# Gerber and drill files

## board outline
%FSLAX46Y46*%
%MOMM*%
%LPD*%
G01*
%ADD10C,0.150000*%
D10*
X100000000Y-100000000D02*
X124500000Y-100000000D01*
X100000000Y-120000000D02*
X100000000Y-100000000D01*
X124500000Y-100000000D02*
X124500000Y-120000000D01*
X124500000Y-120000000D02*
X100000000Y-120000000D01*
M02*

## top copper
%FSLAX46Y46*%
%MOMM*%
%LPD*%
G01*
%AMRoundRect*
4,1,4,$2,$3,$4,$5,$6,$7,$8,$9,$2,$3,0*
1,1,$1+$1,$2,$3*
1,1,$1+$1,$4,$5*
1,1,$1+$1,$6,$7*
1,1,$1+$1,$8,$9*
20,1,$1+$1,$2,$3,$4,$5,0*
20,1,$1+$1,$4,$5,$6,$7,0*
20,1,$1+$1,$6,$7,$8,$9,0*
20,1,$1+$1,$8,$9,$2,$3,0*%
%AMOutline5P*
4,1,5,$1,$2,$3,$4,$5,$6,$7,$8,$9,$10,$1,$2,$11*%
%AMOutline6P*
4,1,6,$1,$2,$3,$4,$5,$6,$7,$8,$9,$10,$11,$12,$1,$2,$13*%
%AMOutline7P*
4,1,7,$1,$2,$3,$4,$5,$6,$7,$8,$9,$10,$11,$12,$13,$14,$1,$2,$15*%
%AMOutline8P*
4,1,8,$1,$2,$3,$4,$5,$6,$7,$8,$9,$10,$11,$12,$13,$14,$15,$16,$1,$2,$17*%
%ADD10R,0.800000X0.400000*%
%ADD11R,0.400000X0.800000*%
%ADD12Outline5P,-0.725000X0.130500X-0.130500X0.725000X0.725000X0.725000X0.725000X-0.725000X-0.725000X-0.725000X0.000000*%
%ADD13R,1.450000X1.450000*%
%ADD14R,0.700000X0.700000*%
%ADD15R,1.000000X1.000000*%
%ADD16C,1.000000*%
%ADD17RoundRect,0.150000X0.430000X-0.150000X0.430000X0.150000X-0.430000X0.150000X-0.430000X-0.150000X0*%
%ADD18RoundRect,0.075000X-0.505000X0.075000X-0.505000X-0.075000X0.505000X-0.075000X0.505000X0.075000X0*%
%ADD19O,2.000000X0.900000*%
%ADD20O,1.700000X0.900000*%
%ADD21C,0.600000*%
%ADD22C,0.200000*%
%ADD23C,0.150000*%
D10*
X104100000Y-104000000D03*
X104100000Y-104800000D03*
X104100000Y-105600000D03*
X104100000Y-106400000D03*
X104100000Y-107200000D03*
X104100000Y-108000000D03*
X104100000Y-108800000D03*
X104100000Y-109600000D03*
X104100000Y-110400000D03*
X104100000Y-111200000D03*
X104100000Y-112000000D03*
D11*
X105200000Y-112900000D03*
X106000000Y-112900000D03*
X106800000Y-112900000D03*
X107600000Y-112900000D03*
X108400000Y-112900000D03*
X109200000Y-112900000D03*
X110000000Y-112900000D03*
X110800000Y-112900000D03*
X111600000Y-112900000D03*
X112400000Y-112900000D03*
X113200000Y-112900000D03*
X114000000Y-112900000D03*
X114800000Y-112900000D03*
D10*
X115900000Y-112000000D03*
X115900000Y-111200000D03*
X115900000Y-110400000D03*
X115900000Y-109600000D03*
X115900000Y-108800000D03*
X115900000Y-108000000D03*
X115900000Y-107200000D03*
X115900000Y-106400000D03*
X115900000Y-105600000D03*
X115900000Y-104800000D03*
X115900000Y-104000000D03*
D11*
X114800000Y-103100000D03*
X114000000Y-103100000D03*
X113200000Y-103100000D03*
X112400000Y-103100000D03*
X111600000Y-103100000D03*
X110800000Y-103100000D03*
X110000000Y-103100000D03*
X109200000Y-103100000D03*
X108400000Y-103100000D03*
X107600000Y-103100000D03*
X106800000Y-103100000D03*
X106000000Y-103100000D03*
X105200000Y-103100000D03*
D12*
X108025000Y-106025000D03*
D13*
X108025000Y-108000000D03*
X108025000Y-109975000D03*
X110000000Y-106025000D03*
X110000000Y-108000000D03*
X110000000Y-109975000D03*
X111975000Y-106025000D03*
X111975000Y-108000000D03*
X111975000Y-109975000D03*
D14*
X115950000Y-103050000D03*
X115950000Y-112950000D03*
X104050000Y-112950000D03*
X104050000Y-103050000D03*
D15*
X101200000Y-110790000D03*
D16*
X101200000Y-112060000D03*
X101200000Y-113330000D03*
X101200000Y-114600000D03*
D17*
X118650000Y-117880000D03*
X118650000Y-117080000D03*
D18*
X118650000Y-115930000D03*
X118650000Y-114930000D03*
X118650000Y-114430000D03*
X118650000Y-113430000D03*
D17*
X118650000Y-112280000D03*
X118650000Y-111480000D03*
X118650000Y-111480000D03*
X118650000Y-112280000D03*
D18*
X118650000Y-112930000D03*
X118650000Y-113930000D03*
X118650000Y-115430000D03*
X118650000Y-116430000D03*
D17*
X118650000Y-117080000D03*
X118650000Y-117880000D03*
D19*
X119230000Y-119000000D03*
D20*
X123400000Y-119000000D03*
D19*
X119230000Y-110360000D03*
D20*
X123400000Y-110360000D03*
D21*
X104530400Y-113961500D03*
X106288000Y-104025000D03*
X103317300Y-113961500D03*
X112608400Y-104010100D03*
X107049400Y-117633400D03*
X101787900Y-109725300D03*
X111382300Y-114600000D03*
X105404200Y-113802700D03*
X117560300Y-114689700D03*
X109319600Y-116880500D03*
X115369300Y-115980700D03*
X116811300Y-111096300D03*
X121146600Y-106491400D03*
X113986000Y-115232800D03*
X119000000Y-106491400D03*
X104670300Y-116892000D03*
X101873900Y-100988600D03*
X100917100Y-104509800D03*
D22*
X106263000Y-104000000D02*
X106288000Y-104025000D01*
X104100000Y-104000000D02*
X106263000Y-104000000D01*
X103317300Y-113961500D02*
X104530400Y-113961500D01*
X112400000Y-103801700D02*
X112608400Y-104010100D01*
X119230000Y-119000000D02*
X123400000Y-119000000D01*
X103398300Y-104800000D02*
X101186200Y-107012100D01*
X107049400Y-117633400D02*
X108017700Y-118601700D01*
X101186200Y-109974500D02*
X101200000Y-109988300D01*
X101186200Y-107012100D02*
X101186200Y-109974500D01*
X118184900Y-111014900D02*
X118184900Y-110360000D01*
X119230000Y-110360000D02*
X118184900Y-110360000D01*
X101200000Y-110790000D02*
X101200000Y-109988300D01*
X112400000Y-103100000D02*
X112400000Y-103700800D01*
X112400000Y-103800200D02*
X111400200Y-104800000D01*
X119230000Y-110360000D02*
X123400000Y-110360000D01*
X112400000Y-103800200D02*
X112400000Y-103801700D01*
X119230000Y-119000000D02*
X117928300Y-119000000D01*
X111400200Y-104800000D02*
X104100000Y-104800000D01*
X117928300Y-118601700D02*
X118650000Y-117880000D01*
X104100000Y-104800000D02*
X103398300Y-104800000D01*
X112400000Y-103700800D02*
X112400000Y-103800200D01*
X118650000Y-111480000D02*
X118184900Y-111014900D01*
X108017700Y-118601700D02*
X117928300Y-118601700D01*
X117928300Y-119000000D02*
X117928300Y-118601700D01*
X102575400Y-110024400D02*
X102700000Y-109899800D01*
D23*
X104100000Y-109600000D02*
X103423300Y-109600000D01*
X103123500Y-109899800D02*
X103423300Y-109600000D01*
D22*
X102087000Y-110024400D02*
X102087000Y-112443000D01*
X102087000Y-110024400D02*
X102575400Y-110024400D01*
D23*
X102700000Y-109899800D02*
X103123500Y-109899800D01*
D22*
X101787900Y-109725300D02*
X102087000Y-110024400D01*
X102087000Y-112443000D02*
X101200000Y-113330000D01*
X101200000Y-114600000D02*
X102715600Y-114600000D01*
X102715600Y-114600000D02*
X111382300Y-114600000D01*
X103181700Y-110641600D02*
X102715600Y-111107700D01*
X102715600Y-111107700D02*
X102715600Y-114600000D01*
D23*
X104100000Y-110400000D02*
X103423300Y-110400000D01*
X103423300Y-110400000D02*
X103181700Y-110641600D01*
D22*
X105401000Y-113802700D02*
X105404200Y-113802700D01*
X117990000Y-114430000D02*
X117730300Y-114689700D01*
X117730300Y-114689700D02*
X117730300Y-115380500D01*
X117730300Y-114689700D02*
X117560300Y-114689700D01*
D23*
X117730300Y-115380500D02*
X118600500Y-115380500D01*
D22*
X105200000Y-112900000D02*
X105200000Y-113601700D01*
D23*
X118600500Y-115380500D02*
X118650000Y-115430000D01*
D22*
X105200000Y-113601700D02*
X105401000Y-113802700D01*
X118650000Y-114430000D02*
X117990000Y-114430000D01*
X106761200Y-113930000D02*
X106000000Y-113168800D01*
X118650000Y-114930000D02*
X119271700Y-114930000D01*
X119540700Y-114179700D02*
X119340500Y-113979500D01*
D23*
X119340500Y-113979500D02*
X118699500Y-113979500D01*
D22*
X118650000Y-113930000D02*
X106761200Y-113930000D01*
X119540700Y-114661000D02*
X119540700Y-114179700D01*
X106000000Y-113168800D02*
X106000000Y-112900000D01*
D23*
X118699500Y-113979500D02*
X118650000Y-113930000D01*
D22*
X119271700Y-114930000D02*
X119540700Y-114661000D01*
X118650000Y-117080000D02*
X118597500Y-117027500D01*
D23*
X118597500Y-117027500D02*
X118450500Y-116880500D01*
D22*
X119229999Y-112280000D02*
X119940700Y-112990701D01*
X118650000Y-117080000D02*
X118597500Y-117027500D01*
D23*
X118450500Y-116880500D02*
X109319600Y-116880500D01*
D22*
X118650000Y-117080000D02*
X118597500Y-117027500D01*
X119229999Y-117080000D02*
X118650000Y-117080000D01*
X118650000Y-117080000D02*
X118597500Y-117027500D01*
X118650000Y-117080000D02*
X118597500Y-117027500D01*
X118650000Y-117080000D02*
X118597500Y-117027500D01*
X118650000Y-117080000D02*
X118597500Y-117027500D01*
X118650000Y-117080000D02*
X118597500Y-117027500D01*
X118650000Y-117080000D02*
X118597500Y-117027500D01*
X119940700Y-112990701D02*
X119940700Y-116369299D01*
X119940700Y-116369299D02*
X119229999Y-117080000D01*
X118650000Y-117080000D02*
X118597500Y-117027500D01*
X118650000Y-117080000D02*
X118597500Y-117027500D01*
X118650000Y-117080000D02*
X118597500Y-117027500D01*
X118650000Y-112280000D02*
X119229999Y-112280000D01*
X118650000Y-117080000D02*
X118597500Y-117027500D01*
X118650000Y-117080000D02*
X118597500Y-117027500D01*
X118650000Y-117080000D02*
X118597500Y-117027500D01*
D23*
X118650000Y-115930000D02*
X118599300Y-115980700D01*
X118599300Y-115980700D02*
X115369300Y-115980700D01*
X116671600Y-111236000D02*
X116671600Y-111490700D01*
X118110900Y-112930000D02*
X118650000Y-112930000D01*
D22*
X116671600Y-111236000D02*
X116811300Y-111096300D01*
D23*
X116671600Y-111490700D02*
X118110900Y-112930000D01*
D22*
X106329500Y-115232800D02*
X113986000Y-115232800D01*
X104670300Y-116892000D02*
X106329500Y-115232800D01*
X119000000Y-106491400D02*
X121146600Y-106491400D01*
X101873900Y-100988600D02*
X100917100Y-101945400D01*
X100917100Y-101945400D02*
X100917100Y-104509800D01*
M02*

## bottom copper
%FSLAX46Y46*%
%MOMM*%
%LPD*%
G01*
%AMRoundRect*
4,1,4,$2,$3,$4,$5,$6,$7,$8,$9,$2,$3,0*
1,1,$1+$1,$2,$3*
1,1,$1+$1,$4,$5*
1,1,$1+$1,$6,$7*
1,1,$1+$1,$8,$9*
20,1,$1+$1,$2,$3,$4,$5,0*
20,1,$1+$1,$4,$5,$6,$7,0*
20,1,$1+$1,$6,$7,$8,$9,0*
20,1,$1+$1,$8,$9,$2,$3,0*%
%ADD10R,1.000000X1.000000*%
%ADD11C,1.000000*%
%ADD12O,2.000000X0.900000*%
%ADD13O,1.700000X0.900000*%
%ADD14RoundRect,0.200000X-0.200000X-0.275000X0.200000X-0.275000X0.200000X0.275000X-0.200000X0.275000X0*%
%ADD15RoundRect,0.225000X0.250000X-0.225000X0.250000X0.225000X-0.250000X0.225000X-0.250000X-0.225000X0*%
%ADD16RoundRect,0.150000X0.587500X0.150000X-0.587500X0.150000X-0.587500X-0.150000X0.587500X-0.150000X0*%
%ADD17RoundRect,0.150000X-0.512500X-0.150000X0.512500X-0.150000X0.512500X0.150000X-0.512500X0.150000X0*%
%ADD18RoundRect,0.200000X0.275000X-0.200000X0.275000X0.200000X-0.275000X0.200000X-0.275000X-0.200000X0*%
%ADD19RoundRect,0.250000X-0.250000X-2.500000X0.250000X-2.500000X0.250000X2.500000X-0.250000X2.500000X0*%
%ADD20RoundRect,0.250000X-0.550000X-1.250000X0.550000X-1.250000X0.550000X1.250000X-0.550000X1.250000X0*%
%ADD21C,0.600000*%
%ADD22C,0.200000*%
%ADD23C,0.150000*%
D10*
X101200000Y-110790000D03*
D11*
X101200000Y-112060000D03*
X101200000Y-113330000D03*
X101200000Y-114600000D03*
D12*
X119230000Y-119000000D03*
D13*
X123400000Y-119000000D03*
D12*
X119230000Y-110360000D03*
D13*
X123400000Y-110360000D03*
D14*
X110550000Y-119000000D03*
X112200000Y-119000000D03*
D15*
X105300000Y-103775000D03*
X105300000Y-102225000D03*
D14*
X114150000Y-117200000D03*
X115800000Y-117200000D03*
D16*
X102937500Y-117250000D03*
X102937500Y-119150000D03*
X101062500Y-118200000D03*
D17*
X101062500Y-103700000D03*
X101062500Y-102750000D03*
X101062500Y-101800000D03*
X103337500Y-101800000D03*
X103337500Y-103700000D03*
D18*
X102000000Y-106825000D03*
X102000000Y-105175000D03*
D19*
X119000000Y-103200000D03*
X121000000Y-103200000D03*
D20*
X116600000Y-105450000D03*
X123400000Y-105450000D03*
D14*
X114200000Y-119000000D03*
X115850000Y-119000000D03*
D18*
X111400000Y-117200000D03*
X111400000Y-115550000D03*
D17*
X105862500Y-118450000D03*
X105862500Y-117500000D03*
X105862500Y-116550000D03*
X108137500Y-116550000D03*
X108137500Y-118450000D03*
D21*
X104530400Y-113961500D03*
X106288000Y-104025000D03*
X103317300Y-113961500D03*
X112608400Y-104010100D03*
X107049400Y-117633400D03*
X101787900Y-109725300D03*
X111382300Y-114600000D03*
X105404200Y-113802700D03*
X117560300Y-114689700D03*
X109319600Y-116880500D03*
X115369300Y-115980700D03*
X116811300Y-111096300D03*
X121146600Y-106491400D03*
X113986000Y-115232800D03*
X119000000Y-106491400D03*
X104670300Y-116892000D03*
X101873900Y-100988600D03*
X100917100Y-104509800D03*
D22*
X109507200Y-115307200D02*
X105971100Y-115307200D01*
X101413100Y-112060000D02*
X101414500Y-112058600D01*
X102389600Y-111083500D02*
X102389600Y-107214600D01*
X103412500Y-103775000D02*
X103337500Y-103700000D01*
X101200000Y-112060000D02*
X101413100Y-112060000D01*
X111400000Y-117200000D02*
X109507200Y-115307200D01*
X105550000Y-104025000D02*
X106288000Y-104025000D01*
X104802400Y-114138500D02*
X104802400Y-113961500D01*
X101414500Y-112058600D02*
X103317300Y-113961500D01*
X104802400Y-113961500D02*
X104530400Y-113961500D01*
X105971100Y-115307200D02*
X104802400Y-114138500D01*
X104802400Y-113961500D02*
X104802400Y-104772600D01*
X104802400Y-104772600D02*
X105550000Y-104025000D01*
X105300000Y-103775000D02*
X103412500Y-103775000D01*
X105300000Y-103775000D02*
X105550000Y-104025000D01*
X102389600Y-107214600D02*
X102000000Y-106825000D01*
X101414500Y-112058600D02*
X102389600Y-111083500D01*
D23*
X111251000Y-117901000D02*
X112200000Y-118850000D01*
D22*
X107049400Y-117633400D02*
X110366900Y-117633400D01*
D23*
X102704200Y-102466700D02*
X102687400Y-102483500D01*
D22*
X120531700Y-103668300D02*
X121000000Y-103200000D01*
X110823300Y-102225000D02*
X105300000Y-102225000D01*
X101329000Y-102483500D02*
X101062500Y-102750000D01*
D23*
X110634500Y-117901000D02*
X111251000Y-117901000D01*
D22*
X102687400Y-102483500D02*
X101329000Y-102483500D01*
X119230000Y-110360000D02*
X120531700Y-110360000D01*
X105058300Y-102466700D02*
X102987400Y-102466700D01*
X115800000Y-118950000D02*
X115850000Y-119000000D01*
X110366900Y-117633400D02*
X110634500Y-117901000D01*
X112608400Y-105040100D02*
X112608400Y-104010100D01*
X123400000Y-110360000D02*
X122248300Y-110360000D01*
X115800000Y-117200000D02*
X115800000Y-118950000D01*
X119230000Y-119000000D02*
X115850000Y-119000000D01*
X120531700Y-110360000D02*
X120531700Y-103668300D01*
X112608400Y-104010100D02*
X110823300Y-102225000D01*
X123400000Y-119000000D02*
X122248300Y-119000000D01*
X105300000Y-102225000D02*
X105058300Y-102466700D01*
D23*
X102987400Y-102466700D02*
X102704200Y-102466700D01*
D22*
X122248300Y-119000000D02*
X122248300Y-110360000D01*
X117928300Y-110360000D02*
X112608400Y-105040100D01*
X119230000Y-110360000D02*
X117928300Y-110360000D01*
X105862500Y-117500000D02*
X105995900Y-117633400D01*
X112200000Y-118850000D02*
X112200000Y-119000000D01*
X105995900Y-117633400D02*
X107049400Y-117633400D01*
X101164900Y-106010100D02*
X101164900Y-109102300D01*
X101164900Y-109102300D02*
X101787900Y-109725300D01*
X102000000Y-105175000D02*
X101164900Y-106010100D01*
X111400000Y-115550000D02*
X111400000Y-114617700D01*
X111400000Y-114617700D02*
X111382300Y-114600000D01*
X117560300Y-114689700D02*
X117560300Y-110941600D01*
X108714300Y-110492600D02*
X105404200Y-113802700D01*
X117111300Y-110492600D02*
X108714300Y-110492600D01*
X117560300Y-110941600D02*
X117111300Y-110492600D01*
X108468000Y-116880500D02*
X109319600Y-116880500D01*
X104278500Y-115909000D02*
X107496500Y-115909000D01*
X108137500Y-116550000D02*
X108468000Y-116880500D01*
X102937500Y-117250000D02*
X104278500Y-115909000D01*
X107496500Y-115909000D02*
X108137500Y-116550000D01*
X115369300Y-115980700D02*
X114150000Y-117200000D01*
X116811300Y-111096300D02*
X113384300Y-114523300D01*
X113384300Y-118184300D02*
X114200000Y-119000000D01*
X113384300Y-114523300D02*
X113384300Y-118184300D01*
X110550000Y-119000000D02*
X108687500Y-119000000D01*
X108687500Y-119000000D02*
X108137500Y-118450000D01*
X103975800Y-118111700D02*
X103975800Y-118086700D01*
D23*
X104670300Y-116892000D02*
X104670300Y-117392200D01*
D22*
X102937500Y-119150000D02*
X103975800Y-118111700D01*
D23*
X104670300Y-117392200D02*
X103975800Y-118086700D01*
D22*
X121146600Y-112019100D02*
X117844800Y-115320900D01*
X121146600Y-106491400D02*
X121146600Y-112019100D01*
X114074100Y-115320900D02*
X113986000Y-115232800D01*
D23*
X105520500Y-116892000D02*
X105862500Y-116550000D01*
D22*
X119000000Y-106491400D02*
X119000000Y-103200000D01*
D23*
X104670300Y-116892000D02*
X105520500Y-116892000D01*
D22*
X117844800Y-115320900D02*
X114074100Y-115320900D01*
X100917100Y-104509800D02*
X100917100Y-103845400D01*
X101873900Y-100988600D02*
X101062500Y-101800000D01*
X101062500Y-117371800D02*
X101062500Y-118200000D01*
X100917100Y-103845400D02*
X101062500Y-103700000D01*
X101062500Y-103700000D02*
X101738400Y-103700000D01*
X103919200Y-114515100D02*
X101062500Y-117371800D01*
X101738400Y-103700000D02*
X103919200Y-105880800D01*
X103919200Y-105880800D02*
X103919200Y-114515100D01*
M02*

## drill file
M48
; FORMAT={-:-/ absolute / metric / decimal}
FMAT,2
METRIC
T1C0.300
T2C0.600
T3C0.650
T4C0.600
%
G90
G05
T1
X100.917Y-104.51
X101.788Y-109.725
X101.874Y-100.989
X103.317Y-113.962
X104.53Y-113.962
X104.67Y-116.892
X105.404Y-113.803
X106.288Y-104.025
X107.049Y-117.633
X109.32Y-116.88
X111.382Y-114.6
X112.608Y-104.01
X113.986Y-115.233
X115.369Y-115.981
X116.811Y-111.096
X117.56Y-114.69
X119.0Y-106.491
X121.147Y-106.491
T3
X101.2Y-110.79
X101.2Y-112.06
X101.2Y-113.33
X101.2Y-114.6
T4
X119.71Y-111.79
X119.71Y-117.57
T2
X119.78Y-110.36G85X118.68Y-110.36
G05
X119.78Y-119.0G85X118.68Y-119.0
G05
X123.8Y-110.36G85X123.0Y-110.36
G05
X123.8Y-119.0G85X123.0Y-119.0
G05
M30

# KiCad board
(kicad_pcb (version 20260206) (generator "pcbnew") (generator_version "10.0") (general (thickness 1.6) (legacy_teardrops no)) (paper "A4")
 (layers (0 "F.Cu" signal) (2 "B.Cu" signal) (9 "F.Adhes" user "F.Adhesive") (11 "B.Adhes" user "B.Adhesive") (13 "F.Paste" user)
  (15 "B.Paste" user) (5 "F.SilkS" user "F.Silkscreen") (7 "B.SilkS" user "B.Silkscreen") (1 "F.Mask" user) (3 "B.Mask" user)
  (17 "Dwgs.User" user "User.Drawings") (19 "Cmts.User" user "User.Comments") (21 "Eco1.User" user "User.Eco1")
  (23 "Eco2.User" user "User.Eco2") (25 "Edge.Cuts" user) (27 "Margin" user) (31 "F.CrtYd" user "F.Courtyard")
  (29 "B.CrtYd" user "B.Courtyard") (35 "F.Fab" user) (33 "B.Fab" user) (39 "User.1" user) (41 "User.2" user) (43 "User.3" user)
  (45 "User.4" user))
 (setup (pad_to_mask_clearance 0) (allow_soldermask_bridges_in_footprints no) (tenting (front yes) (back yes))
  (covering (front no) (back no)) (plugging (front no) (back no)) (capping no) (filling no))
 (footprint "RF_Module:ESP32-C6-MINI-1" (layer "F.Cu") (at 110 108)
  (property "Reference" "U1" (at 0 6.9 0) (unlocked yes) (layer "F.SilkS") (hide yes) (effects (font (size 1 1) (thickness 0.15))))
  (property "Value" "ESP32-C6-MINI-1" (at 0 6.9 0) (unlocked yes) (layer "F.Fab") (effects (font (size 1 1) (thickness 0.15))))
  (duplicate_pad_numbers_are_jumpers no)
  (pad "1" smd rect (at -5.9 -4) (size 0.8 0.4) (layers "F.Cu" "F.Mask" "F.Paste") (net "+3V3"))
  (pad "2" smd rect (at -5.9 -3.2) (size 0.8 0.4) (layers "F.Cu" "F.Mask" "F.Paste") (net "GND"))
  (pad "3" smd rect (at -5.9 -2.4) (size 0.8 0.4) (layers "F.Cu" "F.Mask" "F.Paste"))
  (pad "4" smd rect (at -5.9 -1.6) (size 0.8 0.4) (layers "F.Cu" "F.Mask" "F.Paste"))
  (pad "5" smd rect (at -5.9 -0.8) (size 0.8 0.4) (layers "F.Cu" "F.Mask" "F.Paste"))
  (pad "6" smd rect (at -5.9 0) (size 0.8 0.4) (layers "F.Cu" "F.Mask" "F.Paste"))
  (pad "7" smd rect (at -5.9 0.8) (size 0.8 0.4) (layers "F.Cu" "F.Mask" "F.Paste"))
  (pad "8" smd rect (at -5.9 1.6) (size 0.8 0.4) (layers "F.Cu" "F.Mask" "F.Paste") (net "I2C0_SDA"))
  (pad "9" smd rect (at -5.9 2.4) (size 0.8 0.4) (layers "F.Cu" "F.Mask" "F.Paste") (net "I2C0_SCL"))
  (pad "10" smd rect (at -5.9 3.2) (size 0.8 0.4) (layers "F.Cu" "F.Mask" "F.Paste"))
  (pad "11" smd rect (at -5.9 4) (size 0.8 0.4) (layers "F.Cu" "F.Mask" "F.Paste"))
  (pad "12" smd rect (at -4.8 4.9 90) (size 0.8 0.4) (layers "F.Cu" "F.Mask" "F.Paste") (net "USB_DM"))
  (pad "13" smd rect (at -4 4.9 90) (size 0.8 0.4) (layers "F.Cu" "F.Mask" "F.Paste") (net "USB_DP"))
  (pad "14" smd rect (at -3.2 4.9 90) (size 0.8 0.4) (layers "F.Cu" "F.Mask" "F.Paste"))
  (pad "15" smd rect (at -2.4 4.9 90) (size 0.8 0.4) (layers "F.Cu" "F.Mask" "F.Paste"))
  (pad "16" smd rect (at -1.6 4.9 90) (size 0.8 0.4) (layers "F.Cu" "F.Mask" "F.Paste"))
  (pad "17" smd rect (at -0.8 4.9 90) (size 0.8 0.4) (layers "F.Cu" "F.Mask" "F.Paste"))
  (pad "18" smd rect (at 0 4.9 90) (size 0.8 0.4) (layers "F.Cu" "F.Mask" "F.Paste"))
  (pad "19" smd rect (at 0.8 4.9 90) (size 0.8 0.4) (layers "F.Cu" "F.Mask" "F.Paste"))
  (pad "20" smd rect (at 1.6 4.9 90) (size 0.8 0.4) (layers "F.Cu" "F.Mask" "F.Paste"))
  (pad "21" smd rect (at 2.4 4.9 90) (size 0.8 0.4) (layers "F.Cu" "F.Mask" "F.Paste"))
  (pad "22" smd rect (at 3.2 4.9 90) (size 0.8 0.4) (layers "F.Cu" "F.Mask" "F.Paste"))
  (pad "23" smd rect (at 4 4.9 90) (size 0.8 0.4) (layers "F.Cu" "F.Mask" "F.Paste"))
  (pad "24" smd rect (at 4.8 4.9 90) (size 0.8 0.4) (layers "F.Cu" "F.Mask" "F.Paste"))
  (pad "25" smd rect (at 5.9 4) (size 0.8 0.4) (layers "F.Cu" "F.Mask" "F.Paste"))
  (pad "26" smd rect (at 5.9 3.2) (size 0.8 0.4) (layers "F.Cu" "F.Mask" "F.Paste"))
  (pad "27" smd rect (at 5.9 2.4) (size 0.8 0.4) (layers "F.Cu" "F.Mask" "F.Paste"))
  (pad "28" smd rect (at 5.9 1.6) (size 0.8 0.4) (layers "F.Cu" "F.Mask" "F.Paste"))
  (pad "29" smd rect (at 5.9 0.8) (size 0.8 0.4) (layers "F.Cu" "F.Mask" "F.Paste"))
  (pad "30" smd rect (at 5.9 0) (size 0.8 0.4) (layers "F.Cu" "F.Mask" "F.Paste"))
  (pad "31" smd rect (at 5.9 -0.8) (size 0.8 0.4) (layers "F.Cu" "F.Mask" "F.Paste"))
  (pad "32" smd rect (at 5.9 -1.6) (size 0.8 0.4) (layers "F.Cu" "F.Mask" "F.Paste"))
  (pad "33" smd rect (at 5.9 -2.4) (size 0.8 0.4) (layers "F.Cu" "F.Mask" "F.Paste"))
  (pad "34" smd rect (at 5.9 -3.2) (size 0.8 0.4) (layers "F.Cu" "F.Mask" "F.Paste"))
  (pad "35" smd rect (at 5.9 -4) (size 0.8 0.4) (layers "F.Cu" "F.Mask" "F.Paste"))
  (pad "36" smd rect (at 4.8 -4.9 90) (size 0.8 0.4) (layers "F.Cu" "F.Mask" "F.Paste"))
  (pad "37" smd rect (at 4 -4.9 90) (size 0.8 0.4) (layers "F.Cu" "F.Mask" "F.Paste"))
  (pad "38" smd rect (at 3.2 -4.9 90) (size 0.8 0.4) (layers "F.Cu" "F.Mask" "F.Paste"))
  (pad "39" smd rect (at 2.4 -4.9 90) (size 0.8 0.4) (layers "F.Cu" "F.Mask" "F.Paste") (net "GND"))
  (pad "40" smd rect (at 1.6 -4.9 90) (size 0.8 0.4) (layers "F.Cu" "F.Mask" "F.Paste"))
  (pad "41" smd rect (at 0.8 -4.9 90) (size 0.8 0.4) (layers "F.Cu" "F.Mask" "F.Paste"))
  (pad "42" smd rect (at 0 -4.9 90) (size 0.8 0.4) (layers "F.Cu" "F.Mask" "F.Paste"))
  (pad "43" smd rect (at -0.8 -4.9 90) (size 0.8 0.4) (layers "F.Cu" "F.Mask" "F.Paste"))
  (pad "44" smd rect (at -1.6 -4.9 90) (size 0.8 0.4) (layers "F.Cu" "F.Mask" "F.Paste"))
  (pad "45" smd rect (at -2.4 -4.9 90) (size 0.8 0.4) (layers "F.Cu" "F.Mask" "F.Paste"))
  (pad "46" smd rect (at -3.2 -4.9 90) (size 0.8 0.4) (layers "F.Cu" "F.Mask" "F.Paste"))
  (pad "47" smd rect (at -4 -4.9 90) (size 0.8 0.4) (layers "F.Cu" "F.Mask" "F.Paste"))
  (pad "48" smd rect (at -4.8 -4.9 90) (size 0.8 0.4) (layers "F.Cu" "F.Mask" "F.Paste"))
  (pad "49" smd roundrect (at -1.975 -1.975) (size 1.45 1.45) (layers "F.Cu" "F.Mask" "F.Paste") (roundrect_rratio 0) (chamfer_ratio 0.41)
   (chamfer top_left) (zone_connect 2))
  (pad "49" smd rect (at -1.975 0) (size 1.45 1.45) (layers "F.Cu" "F.Mask" "F.Paste") (zone_connect 2))
  (pad "49" smd rect (at -1.975 1.975) (size 1.45 1.45) (layers "F.Cu" "F.Mask" "F.Paste") (zone_connect 2))
  (pad "49" smd rect (at 0 -1.975) (size 1.45 1.45) (layers "F.Cu" "F.Mask" "F.Paste") (zone_connect 2))
  (pad "49" smd rect (at 0 0) (size 1.45 1.45) (layers "F.Cu" "F.Mask" "F.Paste") (zone_connect 2))
  (pad "49" smd rect (at 0 1.975) (size 1.45 1.45) (layers "F.Cu" "F.Mask" "F.Paste") (zone_connect 2))
  (pad "49" smd rect (at 1.975 -1.975) (size 1.45 1.45) (layers "F.Cu" "F.Mask" "F.Paste") (zone_connect 2))
  (pad "49" smd rect (at 1.975 0) (size 1.45 1.45) (layers "F.Cu" "F.Mask" "F.Paste") (zone_connect 2))
  (pad "49" smd rect (at 1.975 1.975) (size 1.45 1.45) (layers "F.Cu" "F.Mask" "F.Paste") (zone_connect 2))
  (pad "50" smd rect (at 5.95 -4.95) (size 0.7 0.7) (layers "F.Cu" "F.Mask" "F.Paste"))
  (pad "51" smd rect (at 5.95 4.95) (size 0.7 0.7) (layers "F.Cu" "F.Mask" "F.Paste"))
  (pad "52" smd rect (at -5.95 4.95) (size 0.7 0.7) (layers "F.Cu" "F.Mask" "F.Paste"))
  (pad "53" smd rect (at -5.95 -4.95) (size 0.7 0.7) (layers "F.Cu" "F.Mask" "F.Paste")))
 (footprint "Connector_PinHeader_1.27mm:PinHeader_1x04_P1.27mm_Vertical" (layer "F.Cu") (at 101.2 110.79)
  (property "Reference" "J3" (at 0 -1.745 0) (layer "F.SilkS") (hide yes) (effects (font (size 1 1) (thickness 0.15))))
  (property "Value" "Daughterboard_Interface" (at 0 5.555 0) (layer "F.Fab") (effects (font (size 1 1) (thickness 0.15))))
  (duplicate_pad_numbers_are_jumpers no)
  (pad "1" thru_hole rect (at 0 0) (size 1 1) (drill 0.65) (layers "*.Cu" "*.Mask") (remove_unused_layers no) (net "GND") (zone_connect 2))
  (pad "2" thru_hole circle (at 0 1.27) (size 1 1) (drill 0.65) (layers "*.Cu" "*.Mask") (remove_unused_layers no) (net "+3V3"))
  (pad "3" thru_hole circle (at 0 2.54) (size 1 1) (drill 0.65) (layers "*.Cu" "*.Mask") (remove_unused_layers no) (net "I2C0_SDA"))
  (pad "4" thru_hole circle (at 0 3.81) (size 1 1) (drill 0.65) (layers "*.Cu" "*.Mask") (remove_unused_layers no) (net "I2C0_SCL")))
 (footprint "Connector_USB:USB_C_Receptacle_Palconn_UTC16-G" (layer "F.Cu") (at 121.16 114.68 90)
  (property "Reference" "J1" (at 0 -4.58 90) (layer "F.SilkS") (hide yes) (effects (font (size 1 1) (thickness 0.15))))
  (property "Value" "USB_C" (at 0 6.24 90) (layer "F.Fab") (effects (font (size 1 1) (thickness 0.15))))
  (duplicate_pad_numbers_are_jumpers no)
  (pad "" np_thru_hole circle (at -2.89 -1.45 270) (size 0.6 0.6) (drill 0.6) (layers "*.Cu" "*.Mask"))
  (pad "" np_thru_hole circle (at 2.89 -1.45 270) (size 0.6 0.6) (drill 0.6) (layers "*.Cu" "*.Mask"))
  (pad "A1" smd roundrect (at -3.2 -2.51 90) (size 0.6 1.16) (layers "F.Cu" "F.Mask" "F.Paste") (roundrect_rratio 0.25) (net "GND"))
  (pad "A4" smd roundrect (at -2.4 -2.51 90) (size 0.6 1.16) (layers "F.Cu" "F.Mask" "F.Paste") (roundrect_rratio 0.25) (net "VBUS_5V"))
  (pad "A5" smd roundrect (at -1.25 -2.51 270) (size 0.3 1.16) (layers "F.Cu" "F.Mask" "F.Paste") (roundrect_rratio 0.25) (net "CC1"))
  (pad "A6" smd roundrect (at -0.25 -2.51 270) (size 0.3 1.16) (layers "F.Cu" "F.Mask" "F.Paste") (roundrect_rratio 0.25) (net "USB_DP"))
  (pad "A7" smd roundrect (at 0.25 -2.51 270) (size 0.3 1.16) (layers "F.Cu" "F.Mask" "F.Paste") (roundrect_rratio 0.25) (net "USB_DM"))
  (pad "A8" smd roundrect (at 1.25 -2.51 270) (size 0.3 1.16) (layers "F.Cu" "F.Mask" "F.Paste") (roundrect_rratio 0.25))
  (pad "A9" smd roundrect (at 2.4 -2.51 90) (size 0.6 1.16) (layers "F.Cu" "F.Mask" "F.Paste") (roundrect_rratio 0.25) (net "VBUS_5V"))
  (pad "A12" smd roundrect (at 3.2 -2.51 90) (size 0.6 1.16) (layers "F.Cu" "F.Mask" "F.Paste") (roundrect_rratio 0.25) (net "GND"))
  (pad "B1" smd roundrect (at 3.2 -2.51 90) (size 0.6 1.16) (layers "F.Cu" "F.Mask" "F.Paste") (roundrect_rratio 0.25) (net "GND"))
  (pad "B4" smd roundrect (at 2.4 -2.51 90) (size 0.6 1.16) (layers "F.Cu" "F.Mask" "F.Paste") (roundrect_rratio 0.25) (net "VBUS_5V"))
  (pad "B5" smd roundrect (at 1.75 -2.51 270) (size 0.3 1.16) (layers "F.Cu" "F.Mask" "F.Paste") (roundrect_rratio 0.25) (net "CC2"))
  (pad "B6" smd roundrect (at 0.75 -2.51 270) (size 0.3 1.16) (layers "F.Cu" "F.Mask" "F.Paste") (roundrect_rratio 0.25) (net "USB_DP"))
  (pad "B7" smd roundrect (at -0.75 -2.51 270) (size 0.3 1.16) (layers "F.Cu" "F.Mask" "F.Paste") (roundrect_rratio 0.25) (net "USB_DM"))
  (pad "B8" smd roundrect (at -1.75 -2.51 270) (size 0.3 1.16) (layers "F.Cu" "F.Mask" "F.Paste") (roundrect_rratio 0.25))
  (pad "B9" smd roundrect (at -2.4 -2.51 90) (size 0.6 1.16) (layers "F.Cu" "F.Mask" "F.Paste") (roundrect_rratio 0.25) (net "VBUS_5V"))
  (pad "B12" smd roundrect (at -3.2 -2.51 90) (size 0.6 1.16) (layers "F.Cu" "F.Mask" "F.Paste") (roundrect_rratio 0.25) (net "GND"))
  (pad "SH" thru_hole oval (at -4.32 -1.93 180) (size 2 0.9) (drill oval 1.7 0.6) (layers "*.Cu" "*.Mask") (remove_unused_layers no)
   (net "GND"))
  (pad "SH" thru_hole oval (at -4.32 2.24 180) (size 1.7 0.9) (drill oval 1.4 0.6) (layers "*.Cu" "*.Mask") (remove_unused_layers no)
   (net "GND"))
  (pad "SH" thru_hole oval (at 4.32 -1.93 180) (size 2 0.9) (drill oval 1.7 0.6) (layers "*.Cu" "*.Mask") (remove_unused_layers no)
   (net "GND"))
  (pad "SH" thru_hole oval (at 4.32 2.24 180) (size 1.7 0.9) (drill oval 1.4 0.6) (layers "*.Cu" "*.Mask") (remove_unused_layers no)
   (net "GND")))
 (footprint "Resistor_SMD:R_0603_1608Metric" (layer "B.Cu") (at 111.375 119)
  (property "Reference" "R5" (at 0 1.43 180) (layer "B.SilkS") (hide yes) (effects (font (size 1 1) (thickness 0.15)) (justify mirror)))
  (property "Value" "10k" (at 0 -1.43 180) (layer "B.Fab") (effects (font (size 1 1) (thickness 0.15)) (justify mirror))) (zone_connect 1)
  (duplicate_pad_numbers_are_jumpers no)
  (pad "1" smd roundrect (at -0.825 0) (size 0.8 0.95) (layers "B.Cu" "B.Mask" "B.Paste") (roundrect_rratio 0.25) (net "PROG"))
  (pad "2" smd roundrect (at 0.825 0) (size 0.8 0.95) (layers "B.Cu" "B.Mask" "B.Paste") (roundrect_rratio 0.25) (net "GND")))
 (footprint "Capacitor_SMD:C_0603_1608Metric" (layer "B.Cu") (at 105.3 103 90)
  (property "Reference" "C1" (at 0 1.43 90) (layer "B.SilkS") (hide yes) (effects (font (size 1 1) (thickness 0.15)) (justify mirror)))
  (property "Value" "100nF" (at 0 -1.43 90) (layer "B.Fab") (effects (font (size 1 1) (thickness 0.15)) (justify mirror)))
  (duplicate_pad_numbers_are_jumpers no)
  (pad "1" smd roundrect (at -0.775 0 90) (size 0.9 0.95) (layers "B.Cu" "B.Mask" "B.Paste") (roundrect_rratio 0.25) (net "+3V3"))
  (pad "2" smd roundrect (at 0.775 0 90) (size 0.9 0.95) (layers "B.Cu" "B.Mask" "B.Paste") (roundrect_rratio 0.25) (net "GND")))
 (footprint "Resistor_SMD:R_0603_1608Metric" (layer "B.Cu") (at 114.975 117.2)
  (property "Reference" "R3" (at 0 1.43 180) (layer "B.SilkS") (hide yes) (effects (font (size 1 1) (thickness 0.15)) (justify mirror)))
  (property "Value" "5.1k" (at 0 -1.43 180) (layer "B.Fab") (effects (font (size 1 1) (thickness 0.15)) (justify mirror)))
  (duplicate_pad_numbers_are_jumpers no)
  (pad "1" smd roundrect (at -0.825 0) (size 0.8 0.95) (layers "B.Cu" "B.Mask" "B.Paste") (roundrect_rratio 0.25) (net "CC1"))
  (pad "2" smd roundrect (at 0.825 0) (size 0.8 0.95) (layers "B.Cu" "B.Mask" "B.Paste") (roundrect_rratio 0.25) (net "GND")))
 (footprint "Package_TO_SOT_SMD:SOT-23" (layer "B.Cu") (at 102 118.2 180)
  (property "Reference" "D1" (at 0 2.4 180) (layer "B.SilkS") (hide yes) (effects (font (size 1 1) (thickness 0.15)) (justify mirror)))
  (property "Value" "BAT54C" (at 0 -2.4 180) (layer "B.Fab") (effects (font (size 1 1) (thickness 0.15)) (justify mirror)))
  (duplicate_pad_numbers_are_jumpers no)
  (pad "1" smd roundrect (at -0.9375 0.95 180) (size 1.475 0.6) (layers "B.Cu" "B.Mask" "B.Paste") (roundrect_rratio 0.25) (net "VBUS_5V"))
  (pad "2" smd roundrect (at -0.9375 -0.95 180) (size 1.475 0.6) (layers "B.Cu" "B.Mask" "B.Paste") (roundrect_rratio 0.25) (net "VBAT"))
  (pad "3" smd roundrect (at 0.9375 0 180) (size 1.475 0.6) (layers "B.Cu" "B.Mask" "B.Paste") (roundrect_rratio 0.25) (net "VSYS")))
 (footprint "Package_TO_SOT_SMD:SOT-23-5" (layer "B.Cu") (at 102.2 102.75)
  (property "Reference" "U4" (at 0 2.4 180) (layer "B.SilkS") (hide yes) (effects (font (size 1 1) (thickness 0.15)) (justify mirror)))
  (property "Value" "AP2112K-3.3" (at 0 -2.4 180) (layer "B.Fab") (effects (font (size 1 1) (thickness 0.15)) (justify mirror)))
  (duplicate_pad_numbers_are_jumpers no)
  (pad "1" smd roundrect (at -1.1375 0.95) (size 1.325 0.6) (layers "B.Cu" "B.Mask" "B.Paste") (roundrect_rratio 0.25) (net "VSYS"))
  (pad "2" smd roundrect (at -1.1375 0) (size 1.325 0.6) (layers "B.Cu" "B.Mask" "B.Paste") (roundrect_rratio 0.25) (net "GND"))
  (pad "3" smd roundrect (at -1.1375 -0.95) (size 1.325 0.6) (layers "B.Cu" "B.Mask" "B.Paste") (roundrect_rratio 0.25) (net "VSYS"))
  (pad "4" smd roundrect (at 1.1375 -0.95) (size 1.325 0.6) (layers "B.Cu" "B.Mask" "B.Paste") (roundrect_rratio 0.25))
  (pad "5" smd roundrect (at 1.1375 0.95) (size 1.325 0.6) (layers "B.Cu" "B.Mask" "B.Paste") (roundrect_rratio 0.25) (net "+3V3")))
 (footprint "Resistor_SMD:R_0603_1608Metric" (layer "B.Cu") (at 102 106 90)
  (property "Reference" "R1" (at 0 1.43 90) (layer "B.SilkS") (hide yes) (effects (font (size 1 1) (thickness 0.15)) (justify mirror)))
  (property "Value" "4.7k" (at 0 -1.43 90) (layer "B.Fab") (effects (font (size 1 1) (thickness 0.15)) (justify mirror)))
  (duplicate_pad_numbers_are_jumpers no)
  (pad "1" smd roundrect (at -0.825 0 90) (size 0.8 0.95) (layers "B.Cu" "B.Mask" "B.Paste") (roundrect_rratio 0.25) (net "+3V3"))
  (pad "2" smd roundrect (at 0.825 0 90) (size 0.8 0.95) (layers "B.Cu" "B.Mask" "B.Paste") (roundrect_rratio 0.25) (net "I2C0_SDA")))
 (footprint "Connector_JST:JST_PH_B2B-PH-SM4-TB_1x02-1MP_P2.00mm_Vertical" (layer "B.Cu") (at 120 103.7)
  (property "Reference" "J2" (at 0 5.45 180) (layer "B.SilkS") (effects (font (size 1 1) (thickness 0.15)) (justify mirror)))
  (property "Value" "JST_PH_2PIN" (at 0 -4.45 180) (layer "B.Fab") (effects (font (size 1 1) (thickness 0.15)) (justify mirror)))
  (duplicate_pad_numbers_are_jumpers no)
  (pad "1" smd roundrect (at -1 -0.5) (size 1 5.5) (layers "B.Cu" "B.Mask" "B.Paste") (roundrect_rratio 0.25) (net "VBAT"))
  (pad "2" smd roundrect (at 1 -0.5) (size 1 5.5) (layers "B.Cu" "B.Mask" "B.Paste") (roundrect_rratio 0.25) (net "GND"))
  (pad "MP" smd roundrect (at -3.4 1.75) (size 1.6 3) (layers "B.Cu" "B.Mask" "B.Paste") (roundrect_rratio 0.15625))
  (pad "MP" smd roundrect (at 3.4 1.75) (size 1.6 3) (layers "B.Cu" "B.Mask" "B.Paste") (roundrect_rratio 0.15625)))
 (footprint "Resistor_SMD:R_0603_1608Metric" (layer "B.Cu") (at 115.025 119)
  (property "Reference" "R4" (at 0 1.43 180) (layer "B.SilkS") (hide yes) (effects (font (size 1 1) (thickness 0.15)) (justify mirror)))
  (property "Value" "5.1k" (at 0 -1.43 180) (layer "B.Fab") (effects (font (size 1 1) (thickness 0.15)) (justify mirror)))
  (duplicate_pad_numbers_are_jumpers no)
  (pad "1" smd roundrect (at -0.825 0) (size 0.8 0.95) (layers "B.Cu" "B.Mask" "B.Paste") (roundrect_rratio 0.25) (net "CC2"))
  (pad "2" smd roundrect (at 0.825 0) (size 0.8 0.95) (layers "B.Cu" "B.Mask" "B.Paste") (roundrect_rratio 0.25) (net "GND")))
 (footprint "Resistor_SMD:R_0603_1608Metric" (layer "B.Cu") (at 111.4 116.375 90)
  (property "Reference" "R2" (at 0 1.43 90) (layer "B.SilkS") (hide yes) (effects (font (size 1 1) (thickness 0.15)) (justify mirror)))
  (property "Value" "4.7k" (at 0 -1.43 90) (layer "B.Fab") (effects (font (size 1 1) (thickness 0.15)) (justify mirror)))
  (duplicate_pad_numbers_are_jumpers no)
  (pad "1" smd roundrect (at -0.825 0 90) (size 0.8 0.95) (layers "B.Cu" "B.Mask" "B.Paste") (roundrect_rratio 0.25) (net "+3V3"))
  (pad "2" smd roundrect (at 0.825 0 90) (size 0.8 0.95) (layers "B.Cu" "B.Mask" "B.Paste") (roundrect_rratio 0.25) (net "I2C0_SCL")))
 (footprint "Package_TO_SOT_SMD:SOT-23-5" (layer "B.Cu") (at 107 117.5)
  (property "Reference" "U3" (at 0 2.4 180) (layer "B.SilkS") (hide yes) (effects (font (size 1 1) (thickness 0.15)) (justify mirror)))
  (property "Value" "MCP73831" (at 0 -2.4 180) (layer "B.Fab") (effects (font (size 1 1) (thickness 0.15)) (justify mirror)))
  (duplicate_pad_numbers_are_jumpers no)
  (pad "1" smd roundrect (at -1.1375 0.95) (size 1.325 0.6) (layers "B.Cu" "B.Mask" "B.Paste") (roundrect_rratio 0.25))
  (pad "2" smd roundrect (at -1.1375 0) (size 1.325 0.6) (layers "B.Cu" "B.Mask" "B.Paste") (roundrect_rratio 0.25) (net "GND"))
  (pad "3" smd roundrect (at -1.1375 -0.95) (size 1.325 0.6) (layers "B.Cu" "B.Mask" "B.Paste") (roundrect_rratio 0.25) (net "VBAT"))
  (pad "4" smd roundrect (at 1.1375 -0.95) (size 1.325 0.6) (layers "B.Cu" "B.Mask" "B.Paste") (roundrect_rratio 0.25) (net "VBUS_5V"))
  (pad "5" smd roundrect (at 1.1375 0.95) (size 1.325 0.6) (layers "B.Cu" "B.Mask" "B.Paste") (roundrect_rratio 0.25) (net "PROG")))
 (gr_line (start 100 100) (end 124.5 100) (stroke (width 0.15) (type default)) (layer "Edge.Cuts"))
 (gr_line (start 100 120) (end 100 100) (stroke (width 0.15) (type default)) (layer "Edge.Cuts"))
 (gr_line (start 124.5 100) (end 124.5 120) (stroke (width 0.15) (type default)) (layer "Edge.Cuts"))
 (gr_line (start 124.5 120) (end 100 120) (stroke (width 0.15) (type default)) (layer "Edge.Cuts"))
 (segment (start 106.263 104) (end 106.288 104.025) (width 0.2) (layer "F.Cu") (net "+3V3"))
 (segment (start 104.1 104) (end 106.263 104) (width 0.2) (layer "F.Cu") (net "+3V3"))
 (segment (start 103.3173 113.9615) (end 104.5304 113.9615) (width 0.2) (layer "F.Cu") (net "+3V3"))
 (via (at 104.5304 113.9615) (size 0.6) (drill 0.3) (layers "F.Cu" "B.Cu") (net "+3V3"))
 (via (at 106.288 104.025) (size 0.6) (drill 0.3) (layers "F.Cu" "B.Cu") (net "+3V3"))
 (via (at 103.3173 113.9615) (size 0.6) (drill 0.3) (layers "F.Cu" "B.Cu") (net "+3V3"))
 (segment (start 109.5072 115.3072) (end 105.9711 115.3072) (width 0.2) (layer "B.Cu") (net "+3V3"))
 (segment (start 101.4131 112.06) (end 101.4145 112.0586) (width 0.2) (layer "B.Cu") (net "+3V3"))
 (segment (start 102.3896 111.0835) (end 102.3896 107.2146) (width 0.2) (layer "B.Cu") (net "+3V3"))
 (segment (start 103.4125 103.775) (end 103.3375 103.7) (width 0.2) (layer "B.Cu") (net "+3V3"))
 (segment (start 101.2 112.06) (end 101.4131 112.06) (width 0.2) (layer "B.Cu") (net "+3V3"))
 (segment (start 111.4 117.2) (end 109.5072 115.3072) (width 0.2) (layer "B.Cu") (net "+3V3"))
 (segment (start 105.55 104.025) (end 106.288 104.025) (width 0.2) (layer "B.Cu") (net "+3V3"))
 (segment (start 104.8024 114.1385) (end 104.8024 113.9615) (width 0.2) (layer "B.Cu") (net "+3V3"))
 (segment (start 101.4145 112.0586) (end 103.3173 113.9615) (width 0.2) (layer "B.Cu") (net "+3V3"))
 (segment (start 104.8024 113.9615) (end 104.5304 113.9615) (width 0.2) (layer "B.Cu") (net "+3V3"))
 (segment (start 105.9711 115.3072) (end 104.8024 114.1385) (width 0.2) (layer "B.Cu") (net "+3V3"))
 (segment (start 104.8024 113.9615) (end 104.8024 104.7726) (width 0.2) (layer "B.Cu") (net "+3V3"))
 (segment (start 104.8024 104.7726) (end 105.55 104.025) (width 0.2) (layer "B.Cu") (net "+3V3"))
 (segment (start 105.3 103.775) (end 103.4125 103.775) (width 0.2) (layer "B.Cu") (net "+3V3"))
 (segment (start 105.3 103.775) (end 105.55 104.025) (width 0.2) (layer "B.Cu") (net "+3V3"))
 (segment (start 102.3896 107.2146) (end 102 106.825) (width 0.2) (layer "B.Cu") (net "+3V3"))
 (segment (start 101.4145 112.0586) (end 102.3896 111.0835) (width 0.2) (layer "B.Cu") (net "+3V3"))
 (segment (start 112.4 103.8017) (end 112.6084 104.0101) (width 0.2) (layer "F.Cu") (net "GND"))
 (segment (start 119.23 119) (end 123.4 119) (width 0.2) (layer "F.Cu") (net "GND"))
 (segment (start 103.3983 104.8) (end 101.1862 107.0121) (width 0.2) (layer "F.Cu") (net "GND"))
 (segment (start 107.0494 117.6334) (end 108.0177 118.6017) (width 0.2) (layer "F.Cu") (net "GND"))
 (segment (start 101.1862 109.9745) (end 101.2 109.9883) (width 0.2) (layer "F.Cu") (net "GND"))
 (segment (start 101.1862 107.0121) (end 101.1862 109.9745) (width 0.2) (layer "F.Cu") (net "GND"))
 (segment (start 118.1849 111.0149) (end 118.1849 110.36) (width 0.2) (layer "F.Cu") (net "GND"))
 (segment (start 119.23 110.36) (end 118.1849 110.36) (width 0.2) (layer "F.Cu") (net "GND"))
 (segment (start 101.2 110.79) (end 101.2 109.9883) (width 0.2) (layer "F.Cu") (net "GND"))
 (segment (start 112.4 103.1) (end 112.4 103.7008) (width 0.2) (layer "F.Cu") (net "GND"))
 (segment (start 112.4 103.8002) (end 111.4002 104.8) (width 0.2) (layer "F.Cu") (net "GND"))
 (segment (start 119.23 110.36) (end 123.4 110.36) (width 0.2) (layer "F.Cu") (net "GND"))
 (segment (start 112.4 103.8002) (end 112.4 103.8017) (width 0.2) (layer "F.Cu") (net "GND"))
 (segment (start 119.23 119) (end 117.9283 119) (width 0.2) (layer "F.Cu") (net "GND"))
 (segment (start 111.4002 104.8) (end 104.1 104.8) (width 0.2) (layer "F.Cu") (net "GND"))
 (segment (start 117.9283 118.6017) (end 118.65 117.88) (width 0.2) (layer "F.Cu") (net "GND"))
 (segment (start 104.1 104.8) (end 103.3983 104.8) (width 0.2) (layer "F.Cu") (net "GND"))
 (segment (start 112.4 103.7008) (end 112.4 103.8002) (width 0.2) (layer "F.Cu") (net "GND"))
 (segment (start 118.65 111.48) (end 118.1849 111.0149) (width 0.2) (layer "F.Cu") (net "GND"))
 (segment (start 108.0177 118.6017) (end 117.9283 118.6017) (width 0.2) (layer "F.Cu") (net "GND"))
 (segment (start 117.9283 119) (end 117.9283 118.6017) (width 0.2) (layer "F.Cu") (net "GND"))
 (via (at 112.6084 104.0101) (size 0.6) (drill 0.3) (layers "F.Cu" "B.Cu") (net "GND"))
 (via (at 107.0494 117.6334) (size 0.6) (drill 0.3) (layers "F.Cu" "B.Cu") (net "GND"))
 (segment (start 111.251 117.901) (end 112.2 118.85) (width 0.15) (layer "B.Cu") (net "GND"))
 (segment (start 107.0494 117.6334) (end 110.3669 117.6334) (width 0.2) (layer "B.Cu") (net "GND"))
 (segment (start 102.7042 102.4667) (end 102.6874 102.4835) (width 0.15) (layer "B.Cu") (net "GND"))
 (segment (start 120.5317 103.6683) (end 121 103.2) (width 0.2) (layer "B.Cu") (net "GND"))
 (segment (start 110.8233 102.225) (end 105.3 102.225) (width 0.2) (layer "B.Cu") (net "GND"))
 (segment (start 101.329 102.4835) (end 101.0625 102.75) (width 0.2) (layer "B.Cu") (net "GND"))
 (segment (start 110.6345 117.901) (end 111.251 117.901) (width 0.15) (layer "B.Cu") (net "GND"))
 (segment (start 102.6874 102.4835) (end 101.329 102.4835) (width 0.2) (layer "B.Cu") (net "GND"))
 (segment (start 119.23 110.36) (end 120.5317 110.36) (width 0.2) (layer "B.Cu") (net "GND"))
 (segment (start 105.0583 102.4667) (end 102.9874 102.4667) (width 0.2) (layer "B.Cu") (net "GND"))
 (segment (start 115.8 118.95) (end 115.85 119) (width 0.2) (layer "B.Cu") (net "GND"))
 (segment (start 110.3669 117.6334) (end 110.6345 117.901) (width 0.2) (layer "B.Cu") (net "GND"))
 (segment (start 112.6084 105.0401) (end 112.6084 104.0101) (width 0.2) (layer "B.Cu") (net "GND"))
 (segment (start 123.4 110.36) (end 122.2483 110.36) (width 0.2) (layer "B.Cu") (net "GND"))
 (segment (start 115.8 117.2) (end 115.8 118.95) (width 0.2) (layer "B.Cu") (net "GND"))
 (segment (start 119.23 119) (end 115.85 119) (width 0.2) (layer "B.Cu") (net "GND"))
 (segment (start 120.5317 110.36) (end 120.5317 103.6683) (width 0.2) (layer "B.Cu") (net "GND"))
 (segment (start 112.6084 104.0101) (end 110.8233 102.225) (width 0.2) (layer "B.Cu") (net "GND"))
 (segment (start 123.4 119) (end 122.2483 119) (width 0.2) (layer "B.Cu") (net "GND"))
 (segment (start 105.3 102.225) (end 105.0583 102.4667) (width 0.2) (layer "B.Cu") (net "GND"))
 (segment (start 102.9874 102.4667) (end 102.7042 102.4667) (width 0.15) (layer "B.Cu") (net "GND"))
 (segment (start 122.2483 119) (end 122.2483 110.36) (width 0.2) (layer "B.Cu") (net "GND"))
 (segment (start 117.9283 110.36) (end 112.6084 105.0401) (width 0.2) (layer "B.Cu") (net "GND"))
 (segment (start 119.23 110.36) (end 117.9283 110.36) (width 0.2) (layer "B.Cu") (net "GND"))
 (segment (start 105.8625 117.5) (end 105.9959 117.6334) (width 0.2) (layer "B.Cu") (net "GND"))
 (segment (start 112.2 118.85) (end 112.2 119) (width 0.2) (layer "B.Cu") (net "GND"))
 (segment (start 105.9959 117.6334) (end 107.0494 117.6334) (width 0.2) (layer "B.Cu") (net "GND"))
 (segment (start 102.5754 110.0244) (end 102.7 109.8998) (width 0.2) (layer "F.Cu") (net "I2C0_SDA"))
 (segment (start 104.1 109.6) (end 103.4233 109.6) (width 0.15) (layer "F.Cu") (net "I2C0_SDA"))
 (segment (start 103.1235 109.8998) (end 103.4233 109.6) (width 0.15) (layer "F.Cu") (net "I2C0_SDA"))
 (segment (start 102.087 110.0244) (end 102.087 112.443) (width 0.2) (layer "F.Cu") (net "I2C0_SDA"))
 (segment (start 102.087 110.0244) (end 102.5754 110.0244) (width 0.2) (layer "F.Cu") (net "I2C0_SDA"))
 (segment (start 102.7 109.8998) (end 103.1235 109.8998) (width 0.15) (layer "F.Cu") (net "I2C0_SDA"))
 (segment (start 101.7879 109.7253) (end 102.087 110.0244) (width 0.2) (layer "F.Cu") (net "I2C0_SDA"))
 (segment (start 102.087 112.443) (end 101.2 113.33) (width 0.2) (layer "F.Cu") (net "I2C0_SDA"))
 (via (at 101.7879 109.7253) (size 0.6) (drill 0.3) (layers "F.Cu" "B.Cu") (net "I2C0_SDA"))
 (segment (start 101.1649 106.0101) (end 101.1649 109.1023) (width 0.2) (layer "B.Cu") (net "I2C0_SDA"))
 (segment (start 101.1649 109.1023) (end 101.7879 109.7253) (width 0.2) (layer "B.Cu") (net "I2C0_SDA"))
 (segment (start 102 105.175) (end 101.1649 106.0101) (width 0.2) (layer "B.Cu") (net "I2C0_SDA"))
 (segment (start 101.2 114.6) (end 102.7156 114.6) (width 0.2) (layer "F.Cu") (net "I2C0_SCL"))
 (segment (start 102.7156 114.6) (end 111.3823 114.6) (width 0.2) (layer "F.Cu") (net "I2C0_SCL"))
 (segment (start 103.1817 110.6416) (end 102.7156 111.1077) (width 0.2) (layer "F.Cu") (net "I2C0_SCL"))
 (segment (start 102.7156 111.1077) (end 102.7156 114.6) (width 0.2) (layer "F.Cu") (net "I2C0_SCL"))
 (segment (start 104.1 110.4) (end 103.4233 110.4) (width 0.15) (layer "F.Cu") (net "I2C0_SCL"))
 (segment (start 103.4233 110.4) (end 103.1817 110.6416) (width 0.15) (layer "F.Cu") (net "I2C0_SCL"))
 (via (at 111.3823 114.6) (size 0.6) (drill 0.3) (layers "F.Cu" "B.Cu") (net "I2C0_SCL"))
 (segment (start 111.4 115.55) (end 111.4 114.6177) (width 0.2) (layer "B.Cu") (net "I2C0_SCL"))
 (segment (start 111.4 114.6177) (end 111.3823 114.6) (width 0.2) (layer "B.Cu") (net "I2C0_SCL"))
 (segment (start 105.401 113.8027) (end 105.4042 113.8027) (width 0.2) (layer "F.Cu") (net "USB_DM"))
 (segment (start 117.99 114.43) (end 117.7303 114.6897) (width 0.2) (layer "F.Cu") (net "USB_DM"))
 (segment (start 117.7303 114.6897) (end 117.7303 115.3805) (width 0.2) (layer "F.Cu") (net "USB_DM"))
 (segment (start 117.7303 114.6897) (end 117.5603 114.6897) (width 0.2) (layer "F.Cu") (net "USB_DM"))
 (segment (start 117.7303 115.3805) (end 118.6005 115.3805) (width 0.15) (layer "F.Cu") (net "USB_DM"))
 (segment (start 105.2 112.9) (end 105.2 113.6017) (width 0.2) (layer "F.Cu") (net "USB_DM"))
 (segment (start 118.6005 115.3805) (end 118.65 115.43) (width 0.15) (layer "F.Cu") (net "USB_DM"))
 (segment (start 105.2 113.6017) (end 105.401 113.8027) (width 0.2) (layer "F.Cu") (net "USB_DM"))
 (segment (start 118.65 114.43) (end 117.99 114.43) (width 0.2) (layer "F.Cu") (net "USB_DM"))
 (via (at 105.4042 113.8027) (size 0.6) (drill 0.3) (layers "F.Cu" "B.Cu") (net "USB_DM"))
 (via (at 117.5603 114.6897) (size 0.6) (drill 0.3) (layers "F.Cu" "B.Cu") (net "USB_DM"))
 (segment (start 117.5603 114.6897) (end 117.5603 110.9416) (width 0.2) (layer "B.Cu") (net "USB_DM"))
 (segment (start 108.7143 110.4926) (end 105.4042 113.8027) (width 0.2) (layer "B.Cu") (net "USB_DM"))
 (segment (start 117.1113 110.4926) (end 108.7143 110.4926) (width 0.2) (layer "B.Cu") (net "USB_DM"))
 (segment (start 117.5603 110.9416) (end 117.1113 110.4926) (width 0.2) (layer "B.Cu") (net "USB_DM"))
 (segment (start 106.7612 113.93) (end 106 113.1688) (width 0.2) (layer "F.Cu") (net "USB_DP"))
 (segment (start 118.65 114.93) (end 119.2717 114.93) (width 0.2) (layer "F.Cu") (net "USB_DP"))
 (segment (start 119.5407 114.1797) (end 119.3405 113.9795) (width 0.2) (layer "F.Cu") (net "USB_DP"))
 (segment (start 119.3405 113.9795) (end 118.6995 113.9795) (width 0.15) (layer "F.Cu") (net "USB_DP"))
 (segment (start 118.65 113.93) (end 106.7612 113.93) (width 0.2) (layer "F.Cu") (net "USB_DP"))
 (segment (start 119.5407 114.661) (end 119.5407 114.1797) (width 0.2) (layer "F.Cu") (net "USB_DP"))
 (segment (start 106 113.1688) (end 106 112.9) (width 0.2) (layer "F.Cu") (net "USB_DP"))
 (segment (start 118.6995 113.9795) (end 118.65 113.93) (width 0.15) (layer "F.Cu") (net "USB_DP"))
 (segment (start 119.2717 114.93) (end 119.5407 114.661) (width 0.2) (layer "F.Cu") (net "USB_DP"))
 (segment (start 118.65 117.08) (end 118.5975 117.0275) (width 0.2) (layer "F.Cu") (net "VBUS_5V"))
 (segment (start 118.5975 117.0275) (end 118.4505 116.8805) (width 0.15) (layer "F.Cu") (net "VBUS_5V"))
 (segment (start 119.229999 112.28) (end 119.9407 112.990701) (width 0.2) (layer "F.Cu") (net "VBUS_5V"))
 (segment (start 118.65 117.08) (end 118.5975 117.0275) (width 0.2) (layer "F.Cu") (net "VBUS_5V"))
 (segment (start 118.4505 116.8805) (end 109.3196 116.8805) (width 0.15) (layer "F.Cu") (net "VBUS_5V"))
 (segment (start 118.65 117.08) (end 118.5975 117.0275) (width 0.2) (layer "F.Cu") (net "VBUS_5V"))
 (segment (start 119.229999 117.08) (end 118.65 117.08) (width 0.2) (layer "F.Cu") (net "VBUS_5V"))
 (segment (start 118.65 117.08) (end 118.5975 117.0275) (width 0.2) (layer "F.Cu") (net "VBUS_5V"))
 (segment (start 118.65 117.08) (end 118.5975 117.0275) (width 0.2) (layer "F.Cu") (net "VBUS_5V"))
 (segment (start 118.65 117.08) (end 118.5975 117.0275) (width 0.2) (layer "F.Cu") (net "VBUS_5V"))
 (segment (start 118.65 117.08) (end 118.5975 117.0275) (width 0.2) (layer "F.Cu") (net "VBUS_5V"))
 (segment (start 118.65 117.08) (end 118.5975 117.0275) (width 0.2) (layer "F.Cu") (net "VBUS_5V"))
 (segment (start 118.65 117.08) (end 118.5975 117.0275) (width 0.2) (layer "F.Cu") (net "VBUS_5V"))
 (segment (start 119.9407 112.990701) (end 119.9407 116.369299) (width 0.2) (layer "F.Cu") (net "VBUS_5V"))
 (segment (start 119.9407 116.369299) (end 119.229999 117.08) (width 0.2) (layer "F.Cu") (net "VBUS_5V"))
 (segment (start 118.65 117.08) (end 118.5975 117.0275) (width 0.2) (layer "F.Cu") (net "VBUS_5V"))
 (segment (start 118.65 117.08) (end 118.5975 117.0275) (width 0.2) (layer "F.Cu") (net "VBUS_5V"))
 (segment (start 118.65 117.08) (end 118.5975 117.0275) (width 0.2) (layer "F.Cu") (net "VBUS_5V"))
 (segment (start 118.65 112.28) (end 119.229999 112.28) (width 0.2) (layer "F.Cu") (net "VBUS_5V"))
 (segment (start 118.65 117.08) (end 118.5975 117.0275) (width 0.2) (layer "F.Cu") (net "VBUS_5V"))
 (segment (start 118.65 117.08) (end 118.5975 117.0275) (width 0.2) (layer "F.Cu") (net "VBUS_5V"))
 (segment (start 118.65 117.08) (end 118.5975 117.0275) (width 0.2) (layer "F.Cu") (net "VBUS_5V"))
 (via (at 109.3196 116.8805) (size 0.6) (drill 0.3) (layers "F.Cu" "B.Cu") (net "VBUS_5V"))
 (segment (start 108.468 116.8805) (end 109.3196 116.8805) (width 0.2) (layer "B.Cu") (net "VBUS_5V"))
 (segment (start 104.2785 115.909) (end 107.4965 115.909) (width 0.2) (layer "B.Cu") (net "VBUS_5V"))
 (segment (start 108.1375 116.55) (end 108.468 116.8805) (width 0.2) (layer "B.Cu") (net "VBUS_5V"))
 (segment (start 102.9375 117.25) (end 104.2785 115.909) (width 0.2) (layer "B.Cu") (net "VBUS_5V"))
 (segment (start 107.4965 115.909) (end 108.1375 116.55) (width 0.2) (layer "B.Cu") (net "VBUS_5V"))
 (segment (start 118.65 115.93) (end 118.5993 115.9807) (width 0.15) (layer "F.Cu") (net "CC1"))
 (segment (start 118.5993 115.9807) (end 115.3693 115.9807) (width 0.15) (layer "F.Cu") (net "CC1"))
 (via (at 115.3693 115.9807) (size 0.6) (drill 0.3) (layers "F.Cu" "B.Cu") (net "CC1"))
 (segment (start 115.3693 115.9807) (end 114.15 117.2) (width 0.2) (layer "B.Cu") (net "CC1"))
 (segment (start 116.6716 111.236) (end 116.6716 111.4907) (width 0.15) (layer "F.Cu") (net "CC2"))
 (segment (start 118.1109 112.93) (end 118.65 112.93) (width 0.15) (layer "F.Cu") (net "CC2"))
 (segment (start 116.6716 111.236) (end 116.8113 111.0963) (width 0.2) (layer "F.Cu") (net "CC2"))
 (segment (start 116.6716 111.4907) (end 118.1109 112.93) (width 0.15) (layer "F.Cu") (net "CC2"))
 (via (at 116.8113 111.0963) (size 0.6) (drill 0.3) (layers "F.Cu" "B.Cu") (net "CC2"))
 (segment (start 116.8113 111.0963) (end 113.3843 114.5233) (width 0.2) (layer "B.Cu") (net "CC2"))
 (segment (start 113.3843 118.1843) (end 114.2 119) (width 0.2) (layer "B.Cu") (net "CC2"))
 (segment (start 113.3843 114.5233) (end 113.3843 118.1843) (width 0.2) (layer "B.Cu") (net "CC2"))
 (segment (start 110.55 119) (end 108.6875 119) (width 0.2) (layer "B.Cu") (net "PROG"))
 (segment (start 108.6875 119) (end 108.1375 118.45) (width 0.2) (layer "B.Cu") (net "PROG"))
 (segment (start 106.3295 115.2328) (end 113.986 115.2328) (width 0.2) (layer "F.Cu") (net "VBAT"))
 (segment (start 104.6703 116.892) (end 106.3295 115.2328) (width 0.2) (layer "F.Cu") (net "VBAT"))
 (segment (start 119 106.4914) (end 121.1466 106.4914) (width 0.2) (layer "F.Cu") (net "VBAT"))
 (via (at 121.1466 106.4914) (size 0.6) (drill 0.3) (layers "F.Cu" "B.Cu") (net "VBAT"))
 (via (at 113.986 115.2328) (size 0.6) (drill 0.3) (layers "F.Cu" "B.Cu") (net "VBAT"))
 (via (at 119 106.4914) (size 0.6) (drill 0.3) (layers "F.Cu" "B.Cu") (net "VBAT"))
 (via (at 104.6703 116.892) (size 0.6) (drill 0.3) (layers "F.Cu" "B.Cu") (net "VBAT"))
 (segment (start 103.9758 118.1117) (end 103.9758 118.0867) (width 0.2) (layer "B.Cu") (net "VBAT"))
 (segment (start 104.6703 116.892) (end 104.6703 117.3922) (width 0.15) (layer "B.Cu") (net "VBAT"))
 (segment (start 102.9375 119.15) (end 103.9758 118.1117) (width 0.2) (layer "B.Cu") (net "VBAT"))
 (segment (start 104.6703 117.3922) (end 103.9758 118.0867) (width 0.15) (layer "B.Cu") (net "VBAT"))
 (segment (start 121.1466 112.0191) (end 117.8448 115.3209) (width 0.2) (layer "B.Cu") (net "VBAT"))
 (segment (start 121.1466 106.4914) (end 121.1466 112.0191) (width 0.2) (layer "B.Cu") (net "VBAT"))
 (segment (start 114.0741 115.3209) (end 113.986 115.2328) (width 0.2) (layer "B.Cu") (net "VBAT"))
 (segment (start 105.5205 116.892) (end 105.8625 116.55) (width 0.15) (layer "B.Cu") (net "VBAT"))
 (segment (start 119 106.4914) (end 119 103.2) (width 0.2) (layer "B.Cu") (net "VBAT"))
 (segment (start 104.6703 116.892) (end 105.5205 116.892) (width 0.15) (layer "B.Cu") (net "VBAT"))
 (segment (start 117.8448 115.3209) (end 114.0741 115.3209) (width 0.2) (layer "B.Cu") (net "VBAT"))
 (segment (start 101.8739 100.9886) (end 100.9171 101.9454) (width 0.2) (layer "F.Cu") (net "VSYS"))
 (segment (start 100.9171 101.9454) (end 100.9171 104.5098) (width 0.2) (layer "F.Cu") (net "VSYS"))
 (via (at 101.8739 100.9886) (size 0.6) (drill 0.3) (layers "F.Cu" "B.Cu") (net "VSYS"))
 (via (at 100.9171 104.5098) (size 0.6) (drill 0.3) (layers "F.Cu" "B.Cu") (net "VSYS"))
 (segment (start 100.9171 104.5098) (end 100.9171 103.8454) (width 0.2) (layer "B.Cu") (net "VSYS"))
 (segment (start 101.8739 100.9886) (end 101.0625 101.8) (width 0.2) (layer "B.Cu") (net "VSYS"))
 (segment (start 101.0625 117.3718) (end 101.0625 118.2) (width 0.2) (layer "B.Cu") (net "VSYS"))
 (segment (start 100.9171 103.8454) (end 101.0625 103.7) (width 0.2) (layer "B.Cu") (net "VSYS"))
 (segment (start 101.0625 103.7) (end 101.7384 103.7) (width 0.2) (layer "B.Cu") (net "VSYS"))
 (segment (start 103.9192 114.5151) (end 101.0625 117.3718) (width 0.2) (layer "B.Cu") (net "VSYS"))
 (segment (start 101.7384 103.7) (end 103.9192 105.8808) (width 0.2) (layer "B.Cu") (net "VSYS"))
 (segment (start 103.9192 105.8808) (end 103.9192 114.5151) (width 0.2) (layer "B.Cu") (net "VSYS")))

